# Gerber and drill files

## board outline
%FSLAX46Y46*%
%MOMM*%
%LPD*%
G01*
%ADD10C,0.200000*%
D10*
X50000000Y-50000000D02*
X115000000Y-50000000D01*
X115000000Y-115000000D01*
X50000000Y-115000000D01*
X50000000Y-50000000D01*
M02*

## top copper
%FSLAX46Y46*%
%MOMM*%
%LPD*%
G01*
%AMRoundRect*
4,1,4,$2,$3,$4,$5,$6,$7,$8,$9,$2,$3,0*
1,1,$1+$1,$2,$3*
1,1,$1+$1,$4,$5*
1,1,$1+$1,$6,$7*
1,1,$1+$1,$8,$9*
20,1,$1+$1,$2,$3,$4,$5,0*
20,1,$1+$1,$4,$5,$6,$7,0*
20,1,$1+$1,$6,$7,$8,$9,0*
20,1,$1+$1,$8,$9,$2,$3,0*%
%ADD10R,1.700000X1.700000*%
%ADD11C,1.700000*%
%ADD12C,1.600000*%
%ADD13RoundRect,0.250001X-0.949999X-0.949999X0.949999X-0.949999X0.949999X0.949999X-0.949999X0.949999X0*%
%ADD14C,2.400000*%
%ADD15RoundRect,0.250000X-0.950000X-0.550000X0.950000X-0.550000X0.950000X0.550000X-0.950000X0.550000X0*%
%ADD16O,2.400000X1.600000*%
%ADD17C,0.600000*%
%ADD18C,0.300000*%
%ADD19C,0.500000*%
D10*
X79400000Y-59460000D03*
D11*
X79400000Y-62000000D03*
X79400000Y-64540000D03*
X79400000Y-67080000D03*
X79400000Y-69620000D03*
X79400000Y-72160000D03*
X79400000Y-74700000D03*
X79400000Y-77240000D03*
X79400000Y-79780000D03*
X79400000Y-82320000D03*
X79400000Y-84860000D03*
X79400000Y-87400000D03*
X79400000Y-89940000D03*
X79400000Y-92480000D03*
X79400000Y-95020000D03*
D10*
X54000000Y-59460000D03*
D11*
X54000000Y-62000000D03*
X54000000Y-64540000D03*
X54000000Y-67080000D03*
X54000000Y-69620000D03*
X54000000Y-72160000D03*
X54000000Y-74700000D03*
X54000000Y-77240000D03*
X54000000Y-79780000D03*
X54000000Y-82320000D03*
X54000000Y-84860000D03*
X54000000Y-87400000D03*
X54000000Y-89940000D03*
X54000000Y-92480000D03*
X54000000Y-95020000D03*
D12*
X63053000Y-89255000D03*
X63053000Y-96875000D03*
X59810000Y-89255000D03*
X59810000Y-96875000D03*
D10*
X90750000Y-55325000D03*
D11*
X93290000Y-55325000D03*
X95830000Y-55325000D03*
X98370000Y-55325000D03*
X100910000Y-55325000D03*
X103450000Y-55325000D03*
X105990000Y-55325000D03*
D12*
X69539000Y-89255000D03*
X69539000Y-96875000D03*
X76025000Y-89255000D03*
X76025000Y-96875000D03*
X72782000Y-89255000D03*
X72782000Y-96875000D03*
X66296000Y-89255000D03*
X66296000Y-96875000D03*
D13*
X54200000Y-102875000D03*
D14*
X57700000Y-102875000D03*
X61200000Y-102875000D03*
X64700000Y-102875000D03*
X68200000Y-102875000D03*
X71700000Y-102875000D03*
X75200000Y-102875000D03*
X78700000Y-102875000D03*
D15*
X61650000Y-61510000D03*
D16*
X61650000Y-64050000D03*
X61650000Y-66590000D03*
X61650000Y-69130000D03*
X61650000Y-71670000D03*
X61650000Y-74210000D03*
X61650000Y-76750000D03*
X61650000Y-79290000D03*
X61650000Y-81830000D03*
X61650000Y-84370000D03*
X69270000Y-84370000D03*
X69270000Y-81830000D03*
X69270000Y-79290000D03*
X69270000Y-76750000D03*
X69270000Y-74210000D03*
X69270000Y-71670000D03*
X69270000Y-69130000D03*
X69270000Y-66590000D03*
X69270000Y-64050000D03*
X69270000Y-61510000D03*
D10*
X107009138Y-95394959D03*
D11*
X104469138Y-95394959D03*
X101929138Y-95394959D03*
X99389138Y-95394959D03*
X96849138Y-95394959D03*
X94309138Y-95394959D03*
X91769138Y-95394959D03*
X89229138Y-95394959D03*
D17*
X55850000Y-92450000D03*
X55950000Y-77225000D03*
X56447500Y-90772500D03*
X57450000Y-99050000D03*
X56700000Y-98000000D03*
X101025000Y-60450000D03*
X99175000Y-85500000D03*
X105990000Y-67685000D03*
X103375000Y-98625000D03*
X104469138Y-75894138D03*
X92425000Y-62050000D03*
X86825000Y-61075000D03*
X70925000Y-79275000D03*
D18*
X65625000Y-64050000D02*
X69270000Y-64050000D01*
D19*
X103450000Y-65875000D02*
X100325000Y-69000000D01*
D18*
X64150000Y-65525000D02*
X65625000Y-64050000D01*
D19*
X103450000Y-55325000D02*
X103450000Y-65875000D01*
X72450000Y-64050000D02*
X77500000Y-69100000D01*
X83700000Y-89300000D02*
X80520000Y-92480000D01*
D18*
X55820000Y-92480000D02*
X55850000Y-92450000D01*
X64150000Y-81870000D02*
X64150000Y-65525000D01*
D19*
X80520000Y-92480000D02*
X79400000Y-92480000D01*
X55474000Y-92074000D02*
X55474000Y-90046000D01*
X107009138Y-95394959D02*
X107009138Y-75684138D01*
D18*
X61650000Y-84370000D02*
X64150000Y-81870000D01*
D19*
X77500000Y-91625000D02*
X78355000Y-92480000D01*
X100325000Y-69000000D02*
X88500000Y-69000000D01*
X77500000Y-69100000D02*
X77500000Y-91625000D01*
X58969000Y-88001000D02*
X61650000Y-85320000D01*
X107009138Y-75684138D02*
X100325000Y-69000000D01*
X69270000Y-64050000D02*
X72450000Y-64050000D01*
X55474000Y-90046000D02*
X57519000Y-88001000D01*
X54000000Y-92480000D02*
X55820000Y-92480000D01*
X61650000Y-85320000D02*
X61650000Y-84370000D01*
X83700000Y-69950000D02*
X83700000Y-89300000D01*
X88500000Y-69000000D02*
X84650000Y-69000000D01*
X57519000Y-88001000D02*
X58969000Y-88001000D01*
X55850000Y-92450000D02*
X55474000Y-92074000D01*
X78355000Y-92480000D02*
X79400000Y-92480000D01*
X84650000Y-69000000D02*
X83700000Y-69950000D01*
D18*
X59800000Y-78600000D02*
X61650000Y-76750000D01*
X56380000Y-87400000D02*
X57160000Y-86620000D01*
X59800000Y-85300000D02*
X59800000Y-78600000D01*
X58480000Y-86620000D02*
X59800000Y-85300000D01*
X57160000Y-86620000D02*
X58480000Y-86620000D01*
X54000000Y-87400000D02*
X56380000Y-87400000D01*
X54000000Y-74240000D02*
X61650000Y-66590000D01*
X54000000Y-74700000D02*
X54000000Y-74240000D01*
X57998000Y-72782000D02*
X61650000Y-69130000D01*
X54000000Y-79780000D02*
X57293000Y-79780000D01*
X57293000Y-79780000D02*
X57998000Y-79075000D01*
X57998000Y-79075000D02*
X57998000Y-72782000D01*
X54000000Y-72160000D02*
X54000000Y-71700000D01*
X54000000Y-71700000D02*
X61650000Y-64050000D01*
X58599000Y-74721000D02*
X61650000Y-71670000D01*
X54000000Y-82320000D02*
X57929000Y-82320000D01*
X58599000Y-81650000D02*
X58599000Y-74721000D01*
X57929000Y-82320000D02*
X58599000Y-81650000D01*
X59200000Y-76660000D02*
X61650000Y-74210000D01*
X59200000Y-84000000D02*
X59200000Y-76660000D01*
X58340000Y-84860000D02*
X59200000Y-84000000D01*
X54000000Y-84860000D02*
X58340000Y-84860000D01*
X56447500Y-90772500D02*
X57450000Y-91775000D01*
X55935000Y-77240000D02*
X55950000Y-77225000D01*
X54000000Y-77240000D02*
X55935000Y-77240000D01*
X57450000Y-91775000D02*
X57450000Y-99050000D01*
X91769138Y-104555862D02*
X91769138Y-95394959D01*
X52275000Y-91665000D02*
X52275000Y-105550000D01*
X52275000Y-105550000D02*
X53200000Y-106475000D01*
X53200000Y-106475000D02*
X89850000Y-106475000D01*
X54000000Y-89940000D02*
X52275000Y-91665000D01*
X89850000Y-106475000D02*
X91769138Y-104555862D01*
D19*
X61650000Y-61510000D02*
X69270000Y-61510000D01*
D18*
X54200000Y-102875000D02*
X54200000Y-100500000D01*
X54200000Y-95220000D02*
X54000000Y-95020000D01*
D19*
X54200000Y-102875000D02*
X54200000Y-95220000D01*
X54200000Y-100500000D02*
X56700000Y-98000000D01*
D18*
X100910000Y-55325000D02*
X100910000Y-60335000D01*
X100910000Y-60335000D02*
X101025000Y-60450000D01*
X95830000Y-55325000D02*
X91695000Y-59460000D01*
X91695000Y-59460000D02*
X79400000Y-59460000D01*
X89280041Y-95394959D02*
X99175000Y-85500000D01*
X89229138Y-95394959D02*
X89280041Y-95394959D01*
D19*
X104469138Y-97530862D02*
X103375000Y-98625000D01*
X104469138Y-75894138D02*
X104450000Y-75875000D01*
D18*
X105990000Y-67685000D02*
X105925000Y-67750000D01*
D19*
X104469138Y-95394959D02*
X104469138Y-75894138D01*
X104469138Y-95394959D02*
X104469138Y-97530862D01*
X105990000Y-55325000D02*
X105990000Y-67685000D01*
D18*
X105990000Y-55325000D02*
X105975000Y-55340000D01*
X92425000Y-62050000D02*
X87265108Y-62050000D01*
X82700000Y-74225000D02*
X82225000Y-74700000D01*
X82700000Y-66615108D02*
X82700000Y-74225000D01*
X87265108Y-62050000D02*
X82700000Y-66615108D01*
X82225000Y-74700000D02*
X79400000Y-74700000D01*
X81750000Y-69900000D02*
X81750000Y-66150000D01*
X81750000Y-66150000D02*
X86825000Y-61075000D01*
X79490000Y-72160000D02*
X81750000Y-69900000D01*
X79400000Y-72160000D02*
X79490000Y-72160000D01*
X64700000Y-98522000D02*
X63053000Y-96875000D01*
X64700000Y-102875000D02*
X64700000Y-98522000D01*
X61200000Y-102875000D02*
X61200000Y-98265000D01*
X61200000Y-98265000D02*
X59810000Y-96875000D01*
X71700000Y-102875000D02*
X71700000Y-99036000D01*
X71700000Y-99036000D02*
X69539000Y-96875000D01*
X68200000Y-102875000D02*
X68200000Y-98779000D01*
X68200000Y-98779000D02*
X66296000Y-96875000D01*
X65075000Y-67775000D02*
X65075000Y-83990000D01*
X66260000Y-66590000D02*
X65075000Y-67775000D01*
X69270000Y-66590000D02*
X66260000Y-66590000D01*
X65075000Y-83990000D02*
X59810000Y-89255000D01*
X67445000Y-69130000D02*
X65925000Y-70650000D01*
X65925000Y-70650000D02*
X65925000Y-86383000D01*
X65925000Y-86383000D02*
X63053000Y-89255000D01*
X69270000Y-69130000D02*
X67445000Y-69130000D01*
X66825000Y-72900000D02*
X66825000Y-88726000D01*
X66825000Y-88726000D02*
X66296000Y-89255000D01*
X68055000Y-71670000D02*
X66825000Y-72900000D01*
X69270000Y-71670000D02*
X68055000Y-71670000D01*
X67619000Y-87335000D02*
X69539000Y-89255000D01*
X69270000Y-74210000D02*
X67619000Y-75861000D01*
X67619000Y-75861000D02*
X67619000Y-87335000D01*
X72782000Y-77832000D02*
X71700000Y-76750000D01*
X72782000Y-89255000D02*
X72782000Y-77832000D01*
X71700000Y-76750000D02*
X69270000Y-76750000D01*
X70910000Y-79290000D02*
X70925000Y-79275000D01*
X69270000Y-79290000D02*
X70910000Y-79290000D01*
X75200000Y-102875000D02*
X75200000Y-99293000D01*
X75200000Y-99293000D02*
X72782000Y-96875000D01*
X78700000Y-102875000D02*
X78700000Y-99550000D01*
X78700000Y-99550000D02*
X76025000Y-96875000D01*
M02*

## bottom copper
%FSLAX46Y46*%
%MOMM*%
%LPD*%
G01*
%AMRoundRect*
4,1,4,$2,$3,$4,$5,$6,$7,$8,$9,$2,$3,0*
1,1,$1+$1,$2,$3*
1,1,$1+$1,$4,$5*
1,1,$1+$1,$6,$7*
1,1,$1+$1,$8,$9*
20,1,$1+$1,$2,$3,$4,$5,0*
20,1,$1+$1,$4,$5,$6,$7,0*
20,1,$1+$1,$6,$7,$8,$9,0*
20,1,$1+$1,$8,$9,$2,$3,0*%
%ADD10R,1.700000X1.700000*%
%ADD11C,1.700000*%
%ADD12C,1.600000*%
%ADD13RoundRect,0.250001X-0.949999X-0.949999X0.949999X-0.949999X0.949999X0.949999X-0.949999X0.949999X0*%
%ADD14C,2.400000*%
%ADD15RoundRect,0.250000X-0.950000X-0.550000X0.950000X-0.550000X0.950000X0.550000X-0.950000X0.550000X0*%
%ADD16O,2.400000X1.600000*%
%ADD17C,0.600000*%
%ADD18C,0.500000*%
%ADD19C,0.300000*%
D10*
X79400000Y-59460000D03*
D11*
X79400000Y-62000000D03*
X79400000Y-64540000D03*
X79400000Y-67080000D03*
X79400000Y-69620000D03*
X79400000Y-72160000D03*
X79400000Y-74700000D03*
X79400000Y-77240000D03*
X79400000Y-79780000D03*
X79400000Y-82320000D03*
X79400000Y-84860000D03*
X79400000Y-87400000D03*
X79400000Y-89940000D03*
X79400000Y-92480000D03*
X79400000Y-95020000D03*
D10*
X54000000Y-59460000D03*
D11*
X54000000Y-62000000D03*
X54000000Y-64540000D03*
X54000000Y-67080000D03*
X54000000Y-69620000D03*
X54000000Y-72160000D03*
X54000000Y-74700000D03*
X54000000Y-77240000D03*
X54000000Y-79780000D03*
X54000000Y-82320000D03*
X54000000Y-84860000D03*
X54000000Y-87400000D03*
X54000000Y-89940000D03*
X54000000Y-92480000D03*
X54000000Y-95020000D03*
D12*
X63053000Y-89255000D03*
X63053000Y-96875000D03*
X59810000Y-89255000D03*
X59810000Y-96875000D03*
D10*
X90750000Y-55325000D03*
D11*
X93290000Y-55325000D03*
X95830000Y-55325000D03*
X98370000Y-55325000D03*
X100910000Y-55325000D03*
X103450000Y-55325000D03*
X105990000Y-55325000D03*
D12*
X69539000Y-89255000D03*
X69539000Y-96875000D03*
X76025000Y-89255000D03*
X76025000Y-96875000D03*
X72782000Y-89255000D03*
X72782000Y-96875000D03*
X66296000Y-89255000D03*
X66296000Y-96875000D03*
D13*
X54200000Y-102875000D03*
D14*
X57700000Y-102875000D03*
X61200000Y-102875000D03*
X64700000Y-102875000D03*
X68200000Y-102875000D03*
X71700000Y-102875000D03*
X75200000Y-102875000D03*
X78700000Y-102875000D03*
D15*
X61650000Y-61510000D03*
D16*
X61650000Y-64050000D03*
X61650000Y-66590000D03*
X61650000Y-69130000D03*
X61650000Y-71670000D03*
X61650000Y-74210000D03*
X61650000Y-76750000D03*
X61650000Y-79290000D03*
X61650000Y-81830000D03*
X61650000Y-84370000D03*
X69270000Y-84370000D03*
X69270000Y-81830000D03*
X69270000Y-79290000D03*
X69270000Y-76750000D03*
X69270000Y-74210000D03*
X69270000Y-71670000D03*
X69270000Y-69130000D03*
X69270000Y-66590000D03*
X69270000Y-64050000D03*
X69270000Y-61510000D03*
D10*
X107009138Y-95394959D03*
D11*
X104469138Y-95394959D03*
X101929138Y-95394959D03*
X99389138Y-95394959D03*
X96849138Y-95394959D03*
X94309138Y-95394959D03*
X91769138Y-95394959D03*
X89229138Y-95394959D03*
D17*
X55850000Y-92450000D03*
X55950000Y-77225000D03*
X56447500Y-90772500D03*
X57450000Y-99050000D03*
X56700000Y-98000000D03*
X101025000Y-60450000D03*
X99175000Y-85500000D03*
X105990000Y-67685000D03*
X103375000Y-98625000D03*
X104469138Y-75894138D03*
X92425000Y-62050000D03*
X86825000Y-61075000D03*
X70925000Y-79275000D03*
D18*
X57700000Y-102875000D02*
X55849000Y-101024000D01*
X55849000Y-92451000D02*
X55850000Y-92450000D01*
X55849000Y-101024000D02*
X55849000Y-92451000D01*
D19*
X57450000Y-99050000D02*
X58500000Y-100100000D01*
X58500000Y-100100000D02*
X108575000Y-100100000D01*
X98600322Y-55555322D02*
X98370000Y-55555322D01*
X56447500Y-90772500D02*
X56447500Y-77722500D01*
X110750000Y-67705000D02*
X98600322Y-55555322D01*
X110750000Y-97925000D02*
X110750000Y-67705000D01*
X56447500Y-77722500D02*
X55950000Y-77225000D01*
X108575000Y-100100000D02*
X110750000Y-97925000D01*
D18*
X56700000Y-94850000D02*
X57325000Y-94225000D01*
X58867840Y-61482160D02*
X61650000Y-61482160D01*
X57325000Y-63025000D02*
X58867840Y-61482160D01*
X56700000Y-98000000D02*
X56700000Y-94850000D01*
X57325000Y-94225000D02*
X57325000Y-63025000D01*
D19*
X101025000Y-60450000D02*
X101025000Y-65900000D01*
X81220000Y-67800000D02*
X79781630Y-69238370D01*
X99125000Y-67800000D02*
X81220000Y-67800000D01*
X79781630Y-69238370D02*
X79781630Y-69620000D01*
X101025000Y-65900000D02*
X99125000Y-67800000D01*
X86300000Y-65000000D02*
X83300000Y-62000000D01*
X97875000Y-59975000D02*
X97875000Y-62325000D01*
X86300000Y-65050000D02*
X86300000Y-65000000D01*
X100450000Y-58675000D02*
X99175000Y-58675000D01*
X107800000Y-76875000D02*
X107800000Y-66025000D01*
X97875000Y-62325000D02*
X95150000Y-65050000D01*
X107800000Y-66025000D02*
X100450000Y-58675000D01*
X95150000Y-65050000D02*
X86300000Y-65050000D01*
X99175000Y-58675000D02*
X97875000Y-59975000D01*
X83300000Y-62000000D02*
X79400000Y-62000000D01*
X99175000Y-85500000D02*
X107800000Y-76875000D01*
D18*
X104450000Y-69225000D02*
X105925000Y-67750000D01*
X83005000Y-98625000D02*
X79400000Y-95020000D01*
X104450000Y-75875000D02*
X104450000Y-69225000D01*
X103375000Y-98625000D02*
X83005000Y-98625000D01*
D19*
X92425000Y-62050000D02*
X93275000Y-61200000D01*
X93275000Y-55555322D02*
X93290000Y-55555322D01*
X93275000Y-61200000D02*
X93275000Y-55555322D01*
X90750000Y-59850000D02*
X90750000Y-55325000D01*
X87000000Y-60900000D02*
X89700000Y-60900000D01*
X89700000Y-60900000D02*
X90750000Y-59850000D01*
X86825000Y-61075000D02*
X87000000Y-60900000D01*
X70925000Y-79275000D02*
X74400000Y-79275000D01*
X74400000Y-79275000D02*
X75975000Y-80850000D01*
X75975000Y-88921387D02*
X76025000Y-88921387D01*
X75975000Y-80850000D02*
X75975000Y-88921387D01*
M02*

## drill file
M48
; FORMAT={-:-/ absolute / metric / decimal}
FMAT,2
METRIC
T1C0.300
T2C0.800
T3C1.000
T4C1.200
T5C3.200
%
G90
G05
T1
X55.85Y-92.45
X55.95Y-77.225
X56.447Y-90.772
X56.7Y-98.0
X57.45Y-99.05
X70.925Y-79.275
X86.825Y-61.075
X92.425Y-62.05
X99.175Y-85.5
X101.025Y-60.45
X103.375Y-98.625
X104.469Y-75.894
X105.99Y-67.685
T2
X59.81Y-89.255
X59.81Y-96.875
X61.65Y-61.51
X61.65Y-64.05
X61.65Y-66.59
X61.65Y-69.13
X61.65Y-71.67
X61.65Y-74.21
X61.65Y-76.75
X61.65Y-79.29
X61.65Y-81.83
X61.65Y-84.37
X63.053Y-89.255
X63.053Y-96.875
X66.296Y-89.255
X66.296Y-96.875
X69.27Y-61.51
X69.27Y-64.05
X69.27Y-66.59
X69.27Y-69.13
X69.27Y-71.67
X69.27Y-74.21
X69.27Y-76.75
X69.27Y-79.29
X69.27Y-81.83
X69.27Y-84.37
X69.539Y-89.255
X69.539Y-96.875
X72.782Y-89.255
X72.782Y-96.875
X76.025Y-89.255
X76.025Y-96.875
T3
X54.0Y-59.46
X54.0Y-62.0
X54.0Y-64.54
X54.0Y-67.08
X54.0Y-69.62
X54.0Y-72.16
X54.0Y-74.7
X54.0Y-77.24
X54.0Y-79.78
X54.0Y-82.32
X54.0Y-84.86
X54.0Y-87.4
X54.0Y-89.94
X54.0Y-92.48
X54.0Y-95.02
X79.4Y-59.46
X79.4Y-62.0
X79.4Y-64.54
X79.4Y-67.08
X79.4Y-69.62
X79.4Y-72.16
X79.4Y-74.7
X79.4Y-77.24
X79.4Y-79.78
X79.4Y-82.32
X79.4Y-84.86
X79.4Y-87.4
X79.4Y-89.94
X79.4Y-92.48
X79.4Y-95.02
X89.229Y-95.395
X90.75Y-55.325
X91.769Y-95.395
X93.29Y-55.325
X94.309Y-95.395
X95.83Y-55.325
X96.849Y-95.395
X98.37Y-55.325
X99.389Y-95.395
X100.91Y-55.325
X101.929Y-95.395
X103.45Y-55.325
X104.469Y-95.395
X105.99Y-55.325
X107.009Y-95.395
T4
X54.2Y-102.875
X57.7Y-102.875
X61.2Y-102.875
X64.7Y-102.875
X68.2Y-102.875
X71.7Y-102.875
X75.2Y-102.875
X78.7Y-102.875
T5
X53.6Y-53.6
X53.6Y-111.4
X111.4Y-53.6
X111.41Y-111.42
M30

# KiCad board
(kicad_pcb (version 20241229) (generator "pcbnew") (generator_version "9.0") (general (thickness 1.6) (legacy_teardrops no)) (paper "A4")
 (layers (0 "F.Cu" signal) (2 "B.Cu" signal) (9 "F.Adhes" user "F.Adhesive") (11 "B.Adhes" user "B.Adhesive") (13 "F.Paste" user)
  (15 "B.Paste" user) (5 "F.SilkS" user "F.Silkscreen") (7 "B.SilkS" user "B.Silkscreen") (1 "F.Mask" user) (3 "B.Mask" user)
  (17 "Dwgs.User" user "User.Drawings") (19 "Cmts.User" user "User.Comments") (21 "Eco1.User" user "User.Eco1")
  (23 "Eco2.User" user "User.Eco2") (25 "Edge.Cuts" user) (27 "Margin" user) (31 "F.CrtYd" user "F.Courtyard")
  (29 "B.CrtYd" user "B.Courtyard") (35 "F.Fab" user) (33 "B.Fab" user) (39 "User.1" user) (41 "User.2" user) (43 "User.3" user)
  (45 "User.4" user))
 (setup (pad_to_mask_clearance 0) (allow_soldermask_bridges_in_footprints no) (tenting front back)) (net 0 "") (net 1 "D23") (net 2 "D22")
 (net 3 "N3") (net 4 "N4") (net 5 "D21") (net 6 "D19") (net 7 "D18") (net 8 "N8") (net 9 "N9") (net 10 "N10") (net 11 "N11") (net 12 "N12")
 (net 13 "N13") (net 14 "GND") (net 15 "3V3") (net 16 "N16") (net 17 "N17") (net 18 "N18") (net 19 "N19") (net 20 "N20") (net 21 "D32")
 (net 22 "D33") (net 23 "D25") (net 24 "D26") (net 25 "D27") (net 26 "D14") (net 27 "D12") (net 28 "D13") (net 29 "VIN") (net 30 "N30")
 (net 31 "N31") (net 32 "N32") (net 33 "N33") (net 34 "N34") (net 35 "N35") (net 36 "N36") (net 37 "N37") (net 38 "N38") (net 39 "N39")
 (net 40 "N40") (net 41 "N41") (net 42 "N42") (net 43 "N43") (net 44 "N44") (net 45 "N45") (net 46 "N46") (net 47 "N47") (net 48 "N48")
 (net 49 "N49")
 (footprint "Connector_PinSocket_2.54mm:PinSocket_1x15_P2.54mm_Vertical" (layer "F.Cu") (at 79.4 59.46)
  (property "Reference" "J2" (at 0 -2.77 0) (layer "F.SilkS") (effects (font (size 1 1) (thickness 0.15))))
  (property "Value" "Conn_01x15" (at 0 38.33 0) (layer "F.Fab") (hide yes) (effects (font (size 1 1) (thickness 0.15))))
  (pad "1" thru_hole rect (at 0 0) (size 1.7 1.7) (drill 1) (layers "*.Cu" "*.Mask") (remove_unused_layers no) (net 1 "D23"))
  (pad "2" thru_hole circle (at 0 2.54) (size 1.7 1.7) (drill 1) (layers "*.Cu" "*.Mask") (remove_unused_layers no) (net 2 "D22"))
  (pad "3" thru_hole circle (at 0 5.08) (size 1.7 1.7) (drill 1) (layers "*.Cu" "*.Mask") (remove_unused_layers no) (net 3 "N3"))
  (pad "4" thru_hole circle (at 0 7.62) (size 1.7 1.7) (drill 1) (layers "*.Cu" "*.Mask") (remove_unused_layers no) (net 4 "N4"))
  (pad "5" thru_hole circle (at 0 10.16) (size 1.7 1.7) (drill 1) (layers "*.Cu" "*.Mask") (remove_unused_layers no) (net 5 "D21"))
  (pad "6" thru_hole circle (at 0 12.7) (size 1.7 1.7) (drill 1) (layers "*.Cu" "*.Mask") (remove_unused_layers no) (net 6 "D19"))
  (pad "7" thru_hole circle (at 0 15.24) (size 1.7 1.7) (drill 1) (layers "*.Cu" "*.Mask") (remove_unused_layers no) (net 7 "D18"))
  (pad "8" thru_hole circle (at 0 17.78) (size 1.7 1.7) (drill 1) (layers "*.Cu" "*.Mask") (remove_unused_layers no) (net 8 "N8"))
  (pad "9" thru_hole circle (at 0 20.32) (size 1.7 1.7) (drill 1) (layers "*.Cu" "*.Mask") (remove_unused_layers no) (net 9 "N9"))
  (pad "10" thru_hole circle (at 0 22.86) (size 1.7 1.7) (drill 1) (layers "*.Cu" "*.Mask") (remove_unused_layers no) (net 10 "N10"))
  (pad "11" thru_hole circle (at 0 25.4) (size 1.7 1.7) (drill 1) (layers "*.Cu" "*.Mask") (remove_unused_layers no) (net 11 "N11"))
  (pad "12" thru_hole circle (at 0 27.94) (size 1.7 1.7) (drill 1) (layers "*.Cu" "*.Mask") (remove_unused_layers no) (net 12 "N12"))
  (pad "13" thru_hole circle (at 0 30.48) (size 1.7 1.7) (drill 1) (layers "*.Cu" "*.Mask") (remove_unused_layers no) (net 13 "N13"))
  (pad "14" thru_hole circle (at 0 33.02) (size 1.7 1.7) (drill 1) (layers "*.Cu" "*.Mask") (remove_unused_layers no) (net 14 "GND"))
  (pad "15" thru_hole circle (at 0 35.56) (size 1.7 1.7) (drill 1) (layers "*.Cu" "*.Mask") (remove_unused_layers no) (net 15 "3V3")))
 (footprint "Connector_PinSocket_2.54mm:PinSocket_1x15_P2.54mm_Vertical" (layer "F.Cu") (at 54 59.46)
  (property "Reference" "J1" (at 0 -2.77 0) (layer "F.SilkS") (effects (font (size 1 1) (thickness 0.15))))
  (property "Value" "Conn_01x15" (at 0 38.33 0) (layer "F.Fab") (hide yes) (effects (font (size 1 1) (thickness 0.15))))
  (pad "1" thru_hole rect (at 0 0) (size 1.7 1.7) (drill 1) (layers "*.Cu" "*.Mask") (remove_unused_layers no) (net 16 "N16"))
  (pad "2" thru_hole circle (at 0 2.54) (size 1.7 1.7) (drill 1) (layers "*.Cu" "*.Mask") (remove_unused_layers no) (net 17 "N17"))
  (pad "3" thru_hole circle (at 0 5.08) (size 1.7 1.7) (drill 1) (layers "*.Cu" "*.Mask") (remove_unused_layers no) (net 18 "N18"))
  (pad "4" thru_hole circle (at 0 7.62) (size 1.7 1.7) (drill 1) (layers "*.Cu" "*.Mask") (remove_unused_layers no) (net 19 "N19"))
  (pad "5" thru_hole circle (at 0 10.16) (size 1.7 1.7) (drill 1) (layers "*.Cu" "*.Mask") (remove_unused_layers no) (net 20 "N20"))
  (pad "6" thru_hole circle (at 0 12.7) (size 1.7 1.7) (drill 1) (layers "*.Cu" "*.Mask") (remove_unused_layers no) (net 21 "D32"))
  (pad "7" thru_hole circle (at 0 15.24) (size 1.7 1.7) (drill 1) (layers "*.Cu" "*.Mask") (remove_unused_layers no) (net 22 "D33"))
  (pad "8" thru_hole circle (at 0 17.78) (size 1.7 1.7) (drill 1) (layers "*.Cu" "*.Mask") (remove_unused_layers no) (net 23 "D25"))
  (pad "9" thru_hole circle (at 0 20.32) (size 1.7 1.7) (drill 1) (layers "*.Cu" "*.Mask") (remove_unused_layers no) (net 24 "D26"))
  (pad "10" thru_hole circle (at 0 22.86) (size 1.7 1.7) (drill 1) (layers "*.Cu" "*.Mask") (remove_unused_layers no) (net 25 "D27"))
  (pad "11" thru_hole circle (at 0 25.4) (size 1.7 1.7) (drill 1) (layers "*.Cu" "*.Mask") (remove_unused_layers no) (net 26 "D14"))
  (pad "12" thru_hole circle (at 0 27.94) (size 1.7 1.7) (drill 1) (layers "*.Cu" "*.Mask") (remove_unused_layers no) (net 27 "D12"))
  (pad "13" thru_hole circle (at 0 30.48) (size 1.7 1.7) (drill 1) (layers "*.Cu" "*.Mask") (remove_unused_layers no) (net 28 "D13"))
  (pad "14" thru_hole circle (at 0 33.02) (size 1.7 1.7) (drill 1) (layers "*.Cu" "*.Mask") (remove_unused_layers no) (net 14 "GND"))
  (pad "15" thru_hole circle (at 0 35.56) (size 1.7 1.7) (drill 1) (layers "*.Cu" "*.Mask") (remove_unused_layers no) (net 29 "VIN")))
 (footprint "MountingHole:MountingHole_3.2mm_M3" (layer "F.Cu") (at 53.6 53.6)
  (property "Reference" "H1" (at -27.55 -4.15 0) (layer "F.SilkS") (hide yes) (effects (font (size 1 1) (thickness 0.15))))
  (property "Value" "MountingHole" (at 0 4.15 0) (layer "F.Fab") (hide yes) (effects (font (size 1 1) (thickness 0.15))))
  (pad "" np_thru_hole circle (at 0 0) (size 3.2 3.2) (drill 3.2) (layers "*.Cu" "*.Mask")))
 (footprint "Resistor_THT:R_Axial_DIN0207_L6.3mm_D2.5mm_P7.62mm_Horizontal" (layer "F.Cu") (at 63.053 89.255 -90)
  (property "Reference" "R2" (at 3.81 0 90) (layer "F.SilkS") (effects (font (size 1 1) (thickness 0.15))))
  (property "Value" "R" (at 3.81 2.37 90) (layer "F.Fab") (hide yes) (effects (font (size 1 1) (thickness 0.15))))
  (pad "1" thru_hole circle (at 0 0 270) (size 1.6 1.6) (drill 0.8) (layers "*.Cu" "*.Mask") (remove_unused_layers no) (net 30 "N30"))
  (pad "2" thru_hole circle (at 7.62 0 270) (size 1.6 1.6) (drill 0.8) (layers "*.Cu" "*.Mask") (remove_unused_layers no) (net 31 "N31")))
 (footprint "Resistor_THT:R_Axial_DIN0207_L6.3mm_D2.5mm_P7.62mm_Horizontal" (layer "F.Cu") (at 59.81 89.255 -90)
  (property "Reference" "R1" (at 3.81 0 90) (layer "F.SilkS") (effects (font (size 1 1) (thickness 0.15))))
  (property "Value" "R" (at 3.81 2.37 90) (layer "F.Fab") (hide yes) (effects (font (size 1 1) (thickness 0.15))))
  (pad "1" thru_hole circle (at 0 0 270) (size 1.6 1.6) (drill 0.8) (layers "*.Cu" "*.Mask") (remove_unused_layers no) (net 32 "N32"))
  (pad "2" thru_hole circle (at 7.62 0 270) (size 1.6 1.6) (drill 0.8) (layers "*.Cu" "*.Mask") (remove_unused_layers no) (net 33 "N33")))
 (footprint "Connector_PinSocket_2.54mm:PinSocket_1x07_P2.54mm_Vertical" (layer "F.Cu") (at 90.75 55.325 90)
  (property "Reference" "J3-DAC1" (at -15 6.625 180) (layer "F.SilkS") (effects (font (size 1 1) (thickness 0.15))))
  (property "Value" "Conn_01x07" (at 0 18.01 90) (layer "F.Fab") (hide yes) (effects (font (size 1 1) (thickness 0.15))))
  (pad "1" thru_hole rect (at 0 0 90) (size 1.7 1.7) (drill 1) (layers "*.Cu" "*.Mask") (remove_unused_layers no) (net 6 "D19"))
  (pad "2" thru_hole circle (at 0 2.54 90) (size 1.7 1.7) (drill 1) (layers "*.Cu" "*.Mask") (remove_unused_layers no) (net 7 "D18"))
  (pad "3" thru_hole circle (at 0 5.08 90) (size 1.7 1.7) (drill 1) (layers "*.Cu" "*.Mask") (remove_unused_layers no) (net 1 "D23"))
  (pad "4" thru_hole circle (at 0 7.62 90) (size 1.7 1.7) (drill 1) (layers "*.Cu" "*.Mask") (remove_unused_layers no) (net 23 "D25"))
  (pad "5" thru_hole circle (at 0 10.16 90) (size 1.7 1.7) (drill 1) (layers "*.Cu" "*.Mask") (remove_unused_layers no) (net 5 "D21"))
  (pad "6" thru_hole circle (at 0 12.7 90) (size 1.7 1.7) (drill 1) (layers "*.Cu" "*.Mask") (remove_unused_layers no) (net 14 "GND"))
  (pad "7" thru_hole circle (at 0 15.24 90) (size 1.7 1.7) (drill 1) (layers "*.Cu" "*.Mask") (remove_unused_layers no) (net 15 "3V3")))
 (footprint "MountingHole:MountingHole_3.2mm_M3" (layer "F.Cu") (at 53.6 111.4)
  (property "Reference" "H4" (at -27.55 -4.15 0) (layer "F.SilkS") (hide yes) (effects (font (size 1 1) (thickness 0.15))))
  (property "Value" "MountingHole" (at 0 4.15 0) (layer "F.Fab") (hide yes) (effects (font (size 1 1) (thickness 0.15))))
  (pad "" np_thru_hole circle (at 0 0) (size 3.2 3.2) (drill 3.2) (layers "*.Cu" "*.Mask")))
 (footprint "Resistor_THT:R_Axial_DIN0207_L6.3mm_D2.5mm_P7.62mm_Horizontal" (layer "F.Cu") (at 69.539 89.255 -90)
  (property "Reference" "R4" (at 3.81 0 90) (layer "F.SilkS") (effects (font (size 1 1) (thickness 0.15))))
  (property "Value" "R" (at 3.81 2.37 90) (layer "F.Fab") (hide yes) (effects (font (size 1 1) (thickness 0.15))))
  (pad "1" thru_hole circle (at 0 0 270) (size 1.6 1.6) (drill 0.8) (layers "*.Cu" "*.Mask") (remove_unused_layers no) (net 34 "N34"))
  (pad "2" thru_hole circle (at 7.62 0 270) (size 1.6 1.6) (drill 0.8) (layers "*.Cu" "*.Mask") (remove_unused_layers no) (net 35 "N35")))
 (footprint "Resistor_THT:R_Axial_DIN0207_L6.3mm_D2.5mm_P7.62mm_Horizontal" (layer "F.Cu") (at 76.025 89.255 -90)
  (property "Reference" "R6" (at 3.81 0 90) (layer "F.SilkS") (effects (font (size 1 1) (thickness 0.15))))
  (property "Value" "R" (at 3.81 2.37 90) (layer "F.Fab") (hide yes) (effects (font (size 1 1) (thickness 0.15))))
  (pad "1" thru_hole circle (at 0 0 270) (size 1.6 1.6) (drill 0.8) (layers "*.Cu" "*.Mask") (remove_unused_layers no) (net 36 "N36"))
  (pad "2" thru_hole circle (at 7.62 0 270) (size 1.6 1.6) (drill 0.8) (layers "*.Cu" "*.Mask") (remove_unused_layers no) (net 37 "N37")))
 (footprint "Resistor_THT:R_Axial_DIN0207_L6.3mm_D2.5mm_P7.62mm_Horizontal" (layer "F.Cu") (at 72.782 89.255 -90)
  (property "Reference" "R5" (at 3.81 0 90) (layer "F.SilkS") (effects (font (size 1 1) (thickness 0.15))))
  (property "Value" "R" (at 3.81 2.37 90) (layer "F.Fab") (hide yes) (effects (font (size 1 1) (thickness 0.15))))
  (pad "1" thru_hole circle (at 0 0 270) (size 1.6 1.6) (drill 0.8) (layers "*.Cu" "*.Mask") (remove_unused_layers no) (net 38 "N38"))
  (pad "2" thru_hole circle (at 7.62 0 270) (size 1.6 1.6) (drill 0.8) (layers "*.Cu" "*.Mask") (remove_unused_layers no) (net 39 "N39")))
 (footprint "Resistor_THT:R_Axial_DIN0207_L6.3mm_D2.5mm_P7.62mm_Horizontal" (layer "F.Cu") (at 66.296 89.255 -90)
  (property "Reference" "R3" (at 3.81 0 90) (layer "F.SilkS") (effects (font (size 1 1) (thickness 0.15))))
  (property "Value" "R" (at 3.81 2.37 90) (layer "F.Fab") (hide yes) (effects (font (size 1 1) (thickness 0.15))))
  (pad "1" thru_hole circle (at 0 0 270) (size 1.6 1.6) (drill 0.8) (layers "*.Cu" "*.Mask") (remove_unused_layers no) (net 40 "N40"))
  (pad "2" thru_hole circle (at 7.62 0 270) (size 1.6 1.6) (drill 0.8) (layers "*.Cu" "*.Mask") (remove_unused_layers no) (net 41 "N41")))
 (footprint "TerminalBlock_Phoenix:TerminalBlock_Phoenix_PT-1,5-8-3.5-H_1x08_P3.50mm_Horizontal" (layer "F.Cu") (at 54.2 102.875)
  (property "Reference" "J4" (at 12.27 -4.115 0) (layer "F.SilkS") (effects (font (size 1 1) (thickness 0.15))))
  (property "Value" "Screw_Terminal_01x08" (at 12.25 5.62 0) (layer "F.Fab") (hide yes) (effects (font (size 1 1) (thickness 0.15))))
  (pad "1" thru_hole roundrect (at 0 0) (size 2.4 2.4) (drill 1.2) (layers "*.Cu" "*.Mask") (remove_unused_layers no)
   (roundrect_rratio 0.104167) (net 29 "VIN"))
  (pad "2" thru_hole circle (at 3.5 0) (size 2.4 2.4) (drill 1.2) (layers "*.Cu" "*.Mask") (remove_unused_layers no) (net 14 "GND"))
  (pad "3" thru_hole circle (at 7 0) (size 2.4 2.4) (drill 1.2) (layers "*.Cu" "*.Mask") (remove_unused_layers no) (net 33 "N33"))
  (pad "4" thru_hole circle (at 10.5 0) (size 2.4 2.4) (drill 1.2) (layers "*.Cu" "*.Mask") (remove_unused_layers no) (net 31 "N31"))
  (pad "5" thru_hole circle (at 14 0) (size 2.4 2.4) (drill 1.2) (layers "*.Cu" "*.Mask") (remove_unused_layers no) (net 41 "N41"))
  (pad "6" thru_hole circle (at 17.5 0) (size 2.4 2.4) (drill 1.2) (layers "*.Cu" "*.Mask") (remove_unused_layers no) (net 35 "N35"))
  (pad "7" thru_hole circle (at 21 0) (size 2.4 2.4) (drill 1.2) (layers "*.Cu" "*.Mask") (remove_unused_layers no) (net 39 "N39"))
  (pad "8" thru_hole circle (at 24.5 0) (size 2.4 2.4) (drill 1.2) (layers "*.Cu" "*.Mask") (remove_unused_layers no) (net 37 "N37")))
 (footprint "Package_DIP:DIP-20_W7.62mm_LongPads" (layer "F.Cu") (at 61.65 61.51)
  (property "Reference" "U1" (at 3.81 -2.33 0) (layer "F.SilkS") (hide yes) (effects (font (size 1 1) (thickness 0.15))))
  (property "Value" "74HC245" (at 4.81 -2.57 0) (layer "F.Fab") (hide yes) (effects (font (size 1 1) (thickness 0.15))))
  (pad "1" thru_hole roundrect (at 0 0) (size 2.4 1.6) (drill 0.8) (layers "*.Cu" "*.Mask") (remove_unused_layers no)
   (roundrect_rratio 0.15625) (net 29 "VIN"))
  (pad "2" thru_hole oval (at 0 2.54) (size 2.4 1.6) (drill 0.8) (layers "*.Cu" "*.Mask") (remove_unused_layers no) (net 21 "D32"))
  (pad "3" thru_hole oval (at 0 5.08) (size 2.4 1.6) (drill 0.8) (layers "*.Cu" "*.Mask") (remove_unused_layers no) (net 22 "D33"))
  (pad "4" thru_hole oval (at 0 7.62) (size 2.4 1.6) (drill 0.8) (layers "*.Cu" "*.Mask") (remove_unused_layers no) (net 24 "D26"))
  (pad "5" thru_hole oval (at 0 10.16) (size 2.4 1.6) (drill 0.8) (layers "*.Cu" "*.Mask") (remove_unused_layers no) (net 25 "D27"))
  (pad "6" thru_hole oval (at 0 12.7) (size 2.4 1.6) (drill 0.8) (layers "*.Cu" "*.Mask") (remove_unused_layers no) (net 26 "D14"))
  (pad "7" thru_hole oval (at 0 15.24) (size 2.4 1.6) (drill 0.8) (layers "*.Cu" "*.Mask") (remove_unused_layers no) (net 27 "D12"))
  (pad "8" thru_hole oval (at 0 17.78) (size 2.4 1.6) (drill 0.8) (layers "*.Cu" "*.Mask") (remove_unused_layers no) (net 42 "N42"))
  (pad "9" thru_hole oval (at 0 20.32) (size 2.4 1.6) (drill 0.8) (layers "*.Cu" "*.Mask") (remove_unused_layers no) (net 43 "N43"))
  (pad "10" thru_hole oval (at 0 22.86) (size 2.4 1.6) (drill 0.8) (layers "*.Cu" "*.Mask") (remove_unused_layers no) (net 14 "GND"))
  (pad "11" thru_hole oval (at 7.62 22.86) (size 2.4 1.6) (drill 0.8) (layers "*.Cu" "*.Mask") (remove_unused_layers no) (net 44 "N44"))
  (pad "12" thru_hole oval (at 7.62 20.32) (size 2.4 1.6) (drill 0.8) (layers "*.Cu" "*.Mask") (remove_unused_layers no) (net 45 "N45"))
  (pad "13" thru_hole oval (at 7.62 17.78) (size 2.4 1.6) (drill 0.8) (layers "*.Cu" "*.Mask") (remove_unused_layers no) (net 36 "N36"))
  (pad "14" thru_hole oval (at 7.62 15.24) (size 2.4 1.6) (drill 0.8) (layers "*.Cu" "*.Mask") (remove_unused_layers no) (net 38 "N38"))
  (pad "15" thru_hole oval (at 7.62 12.7) (size 2.4 1.6) (drill 0.8) (layers "*.Cu" "*.Mask") (remove_unused_layers no) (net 34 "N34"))
  (pad "16" thru_hole oval (at 7.62 10.16) (size 2.4 1.6) (drill 0.8) (layers "*.Cu" "*.Mask") (remove_unused_layers no) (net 40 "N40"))
  (pad "17" thru_hole oval (at 7.62 7.62) (size 2.4 1.6) (drill 0.8) (layers "*.Cu" "*.Mask") (remove_unused_layers no) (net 30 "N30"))
  (pad "18" thru_hole oval (at 7.62 5.08) (size 2.4 1.6) (drill 0.8) (layers "*.Cu" "*.Mask") (remove_unused_layers no) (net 32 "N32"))
  (pad "19" thru_hole oval (at 7.62 2.54) (size 2.4 1.6) (drill 0.8) (layers "*.Cu" "*.Mask") (remove_unused_layers no) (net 14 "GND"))
  (pad "20" thru_hole oval (at 7.62 0) (size 2.4 1.6) (drill 0.8) (layers "*.Cu" "*.Mask") (remove_unused_layers no) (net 29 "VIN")))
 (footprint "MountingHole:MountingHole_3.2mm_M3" (layer "F.Cu") (at 111.41 111.42)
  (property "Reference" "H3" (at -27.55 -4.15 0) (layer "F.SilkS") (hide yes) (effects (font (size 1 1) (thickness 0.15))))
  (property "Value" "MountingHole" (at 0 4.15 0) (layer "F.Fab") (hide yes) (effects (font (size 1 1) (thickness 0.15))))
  (pad "" np_thru_hole circle (at 0 0) (size 3.2 3.2) (drill 3.2) (layers "*.Cu" "*.Mask")))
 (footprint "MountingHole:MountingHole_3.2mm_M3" (layer "F.Cu") (at 111.4 53.6)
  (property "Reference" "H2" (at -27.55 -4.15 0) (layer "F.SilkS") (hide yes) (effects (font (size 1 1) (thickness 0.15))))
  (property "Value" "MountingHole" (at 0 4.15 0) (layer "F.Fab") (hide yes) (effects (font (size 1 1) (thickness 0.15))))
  (pad "" np_thru_hole circle (at 0 0) (size 3.2 3.2) (drill 3.2) (layers "*.Cu" "*.Mask")))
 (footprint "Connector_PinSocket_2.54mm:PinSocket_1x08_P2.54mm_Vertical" (layer "F.Cu") (at 107.009138 95.394959 -90)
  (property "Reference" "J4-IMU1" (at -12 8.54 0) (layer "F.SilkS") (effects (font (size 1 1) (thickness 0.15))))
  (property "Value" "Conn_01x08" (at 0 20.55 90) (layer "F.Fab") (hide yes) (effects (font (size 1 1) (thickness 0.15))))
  (pad "1" thru_hole rect (at 0 0 270) (size 1.7 1.7) (drill 1) (layers "*.Cu" "*.Mask") (remove_unused_layers no) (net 14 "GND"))
  (pad "2" thru_hole circle (at 0 2.54 270) (size 1.7 1.7) (drill 1) (layers "*.Cu" "*.Mask") (remove_unused_layers no) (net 15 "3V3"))
  (pad "3" thru_hole circle (at 0 5.08 270) (size 1.7 1.7) (drill 1) (layers "*.Cu" "*.Mask") (remove_unused_layers no) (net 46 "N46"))
  (pad "4" thru_hole circle (at 0 7.62 270) (size 1.7 1.7) (drill 1) (layers "*.Cu" "*.Mask") (remove_unused_layers no) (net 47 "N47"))
  (pad "5" thru_hole circle (at 0 10.16 270) (size 1.7 1.7) (drill 1) (layers "*.Cu" "*.Mask") (remove_unused_layers no) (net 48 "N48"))
  (pad "6" thru_hole circle (at 0 12.7 270) (size 1.7 1.7) (drill 1) (layers "*.Cu" "*.Mask") (remove_unused_layers no) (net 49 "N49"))
  (pad "7" thru_hole circle (at 0 15.24 270) (size 1.7 1.7) (drill 1) (layers "*.Cu" "*.Mask") (remove_unused_layers no) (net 28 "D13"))
  (pad "8" thru_hole circle (at 0 17.78 270) (size 1.7 1.7) (drill 1) (layers "*.Cu" "*.Mask") (remove_unused_layers no) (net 2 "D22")))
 (gr_rect (start 50 50) (end 115 115) (stroke (width 0.2) (type solid)) (fill no) (layer "Edge.Cuts"))
 (segment (start 65.625 64.05) (end 69.27 64.05) (width 0.3) (layer "F.Cu") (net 14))
 (segment (start 103.45 65.875) (end 100.325 69) (width 0.5) (layer "F.Cu") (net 14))
 (segment (start 64.15 65.525) (end 65.625 64.05) (width 0.3) (layer "F.Cu") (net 14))
 (segment (start 103.45 55.325) (end 103.45 65.875) (width 0.5) (layer "F.Cu") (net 14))
 (segment (start 72.45 64.05) (end 77.5 69.1) (width 0.5) (layer "F.Cu") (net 14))
 (segment (start 83.7 89.3) (end 80.52 92.48) (width 0.5) (layer "F.Cu") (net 14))
 (segment (start 55.82 92.48) (end 55.85 92.45) (width 0.3) (layer "F.Cu") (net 14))
 (segment (start 64.15 81.87) (end 64.15 65.525) (width 0.3) (layer "F.Cu") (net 14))
 (segment (start 80.52 92.48) (end 79.4 92.48) (width 0.5) (layer "F.Cu") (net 14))
 (segment (start 55.474 92.074) (end 55.474 90.046) (width 0.5) (layer "F.Cu") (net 14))
 (segment (start 107.009138 95.394959) (end 107.009138 75.684138) (width 0.5) (layer "F.Cu") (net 14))
 (segment (start 61.65 84.37) (end 64.15 81.87) (width 0.3) (layer "F.Cu") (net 14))
 (segment (start 77.5 91.625) (end 78.355 92.48) (width 0.5) (layer "F.Cu") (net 14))
 (segment (start 100.325 69) (end 88.5 69) (width 0.5) (layer "F.Cu") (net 14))
 (segment (start 77.5 69.1) (end 77.5 91.625) (width 0.5) (layer "F.Cu") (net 14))
 (segment (start 58.969 88.001) (end 61.65 85.32) (width 0.5) (layer "F.Cu") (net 14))
 (segment (start 107.009138 75.684138) (end 100.325 69) (width 0.5) (layer "F.Cu") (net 14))
 (segment (start 69.27 64.05) (end 72.45 64.05) (width 0.5) (layer "F.Cu") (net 14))
 (segment (start 55.474 90.046) (end 57.519 88.001) (width 0.5) (layer "F.Cu") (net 14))
 (segment (start 54 92.48) (end 55.82 92.48) (width 0.5) (layer "F.Cu") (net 14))
 (segment (start 61.65 85.32) (end 61.65 84.37) (width 0.5) (layer "F.Cu") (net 14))
 (segment (start 83.7 69.95) (end 83.7 89.3) (width 0.5) (layer "F.Cu") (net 14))
 (segment (start 88.5 69) (end 84.65 69) (width 0.5) (layer "F.Cu") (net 14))
 (segment (start 57.519 88.001) (end 58.969 88.001) (width 0.5) (layer "F.Cu") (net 14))
 (segment (start 55.85 92.45) (end 55.474 92.074) (width 0.5) (layer "F.Cu") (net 14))
 (segment (start 78.355 92.48) (end 79.4 92.48) (width 0.5) (layer "F.Cu") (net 14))
 (segment (start 84.65 69) (end 83.7 69.95) (width 0.5) (layer "F.Cu") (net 14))
 (via (at 55.85 92.45) (size 0.6) (drill 0.3) (layers "F.Cu" "B.Cu") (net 14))
 (segment (start 57.7 102.875) (end 55.849 101.024) (width 0.5) (layer "B.Cu") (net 14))
 (segment (start 55.849 92.451) (end 55.85 92.45) (width 0.5) (layer "B.Cu") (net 14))
 (segment (start 55.849 101.024) (end 55.849 92.451) (width 0.5) (layer "B.Cu") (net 14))
 (segment (start 59.8 78.6) (end 61.65 76.75) (width 0.3) (layer "F.Cu") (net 27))
 (segment (start 56.38 87.4) (end 57.16 86.62) (width 0.3) (layer "F.Cu") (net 27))
 (segment (start 59.8 85.3) (end 59.8 78.6) (width 0.3) (layer "F.Cu") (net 27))
 (segment (start 58.48 86.62) (end 59.8 85.3) (width 0.3) (layer "F.Cu") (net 27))
 (segment (start 57.16 86.62) (end 58.48 86.62) (width 0.3) (layer "F.Cu") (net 27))
 (segment (start 54 87.4) (end 56.38 87.4) (width 0.3) (layer "F.Cu") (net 27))
 (segment (start 54 74.24) (end 61.65 66.59) (width 0.3) (layer "F.Cu") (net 22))
 (segment (start 54 74.7) (end 54 74.24) (width 0.3) (layer "F.Cu") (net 22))
 (segment (start 57.998 72.782) (end 61.65 69.13) (width 0.3) (layer "F.Cu") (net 24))
 (segment (start 54 79.78) (end 57.293 79.78) (width 0.3) (layer "F.Cu") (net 24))
 (segment (start 57.293 79.78) (end 57.998 79.075) (width 0.3) (layer "F.Cu") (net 24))
 (segment (start 57.998 79.075) (end 57.998 72.782) (width 0.3) (layer "F.Cu") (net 24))
 (segment (start 54 72.16) (end 54 71.7) (width 0.3) (layer "F.Cu") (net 21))
 (segment (start 54 71.7) (end 61.65 64.05) (width 0.3) (layer "F.Cu") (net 21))
 (segment (start 58.599 74.721) (end 61.65 71.67) (width 0.3) (layer "F.Cu") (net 25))
 (segment (start 54 82.32) (end 57.929 82.32) (width 0.3) (layer "F.Cu") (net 25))
 (segment (start 58.599 81.65) (end 58.599 74.721) (width 0.3) (layer "F.Cu") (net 25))
 (segment (start 57.929 82.32) (end 58.599 81.65) (width 0.3) (layer "F.Cu") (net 25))
 (segment (start 59.2 76.66) (end 61.65 74.21) (width 0.3) (layer "F.Cu") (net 26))
 (segment (start 59.2 84) (end 59.2 76.66) (width 0.3) (layer "F.Cu") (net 26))
 (segment (start 58.34 84.86) (end 59.2 84) (width 0.3) (layer "F.Cu") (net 26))
 (segment (start 54 84.86) (end 58.34 84.86) (width 0.3) (layer "F.Cu") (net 26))
 (segment (start 56.4475 90.7725) (end 57.45 91.775) (width 0.3) (layer "F.Cu") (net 23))
 (segment (start 55.935 77.24) (end 55.95 77.225) (width 0.3) (layer "F.Cu") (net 23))
 (segment (start 54 77.24) (end 55.935 77.24) (width 0.3) (layer "F.Cu") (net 23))
 (segment (start 57.45 91.775) (end 57.45 99.05) (width 0.3) (layer "F.Cu") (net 23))
 (via (at 55.95 77.225) (size 0.6) (drill 0.3) (layers "F.Cu" "B.Cu") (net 23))
 (via (at 56.4475 90.7725) (size 0.6) (drill 0.3) (layers "F.Cu" "B.Cu") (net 23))
 (via (at 57.45 99.05) (size 0.6) (drill 0.3) (layers "F.Cu" "B.Cu") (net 23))
 (segment (start 57.45 99.05) (end 58.5 100.1) (width 0.3) (layer "B.Cu") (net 23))
 (segment (start 58.5 100.1) (end 108.575 100.1) (width 0.3) (layer "B.Cu") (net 23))
 (segment (start 98.600322 55.555322) (end 98.37 55.555322) (width 0.3) (layer "B.Cu") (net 23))
 (segment (start 56.4475 90.7725) (end 56.4475 77.7225) (width 0.3) (layer "B.Cu") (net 23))
 (segment (start 110.75 67.705) (end 98.600322 55.555322) (width 0.3) (layer "B.Cu") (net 23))
 (segment (start 110.75 97.925) (end 110.75 67.705) (width 0.3) (layer "B.Cu") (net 23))
 (segment (start 56.4475 77.7225) (end 55.95 77.225) (width 0.3) (layer "B.Cu") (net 23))
 (segment (start 108.575 100.1) (end 110.75 97.925) (width 0.3) (layer "B.Cu") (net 23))
 (segment (start 91.769138 104.555862) (end 91.769138 95.394959) (width 0.3) (layer "F.Cu") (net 28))
 (segment (start 52.275 91.665) (end 52.275 105.55) (width 0.3) (layer "F.Cu") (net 28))
 (segment (start 52.275 105.55) (end 53.2 106.475) (width 0.3) (layer "F.Cu") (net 28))
 (segment (start 53.2 106.475) (end 89.85 106.475) (width 0.3) (layer "F.Cu") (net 28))
 (segment (start 54 89.94) (end 52.275 91.665) (width 0.3) (layer "F.Cu") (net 28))
 (segment (start 89.85 106.475) (end 91.769138 104.555862) (width 0.3) (layer "F.Cu") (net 28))
 (segment (start 61.65 61.51) (end 69.27 61.51) (width 0.5) (layer "F.Cu") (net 29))
 (segment (start 54.2 102.875) (end 54.2 100.5) (width 0.3) (layer "F.Cu") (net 29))
 (segment (start 54.2 95.22) (end 54 95.02) (width 0.3) (layer "F.Cu") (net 29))
 (segment (start 54.2 102.875) (end 54.2 95.22) (width 0.5) (layer "F.Cu") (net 29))
 (segment (start 54.2 100.5) (end 56.7 98) (width 0.5) (layer "F.Cu") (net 29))
 (via (at 56.7 98) (size 0.6) (drill 0.3) (layers "F.Cu" "B.Cu") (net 29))
 (segment (start 56.7 94.85) (end 57.325 94.225) (width 0.5) (layer "B.Cu") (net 29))
 (segment (start 58.86784 61.48216) (end 61.65 61.48216) (width 0.5) (layer "B.Cu") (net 29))
 (segment (start 57.325 63.025) (end 58.86784 61.48216) (width 0.5) (layer "B.Cu") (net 29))
 (segment (start 56.7 98) (end 56.7 94.85) (width 0.5) (layer "B.Cu") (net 29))
 (segment (start 57.325 94.225) (end 57.325 63.025) (width 0.5) (layer "B.Cu") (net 29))
 (segment (start 100.91 55.325) (end 100.91 60.335) (width 0.3) (layer "F.Cu") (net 5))
 (segment (start 100.91 60.335) (end 101.025 60.45) (width 0.3) (layer "F.Cu") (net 5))
 (via (at 101.025 60.45) (size 0.6) (drill 0.3) (layers "F.Cu" "B.Cu") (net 5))
 (segment (start 101.025 60.45) (end 101.025 65.9) (width 0.3) (layer "B.Cu") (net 5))
 (segment (start 81.22 67.8) (end 79.78163 69.23837) (width 0.3) (layer "B.Cu") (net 5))
 (segment (start 99.125 67.8) (end 81.22 67.8) (width 0.3) (layer "B.Cu") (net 5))
 (segment (start 79.78163 69.23837) (end 79.78163 69.62) (width 0.3) (layer "B.Cu") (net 5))
 (segment (start 101.025 65.9) (end 99.125 67.8) (width 0.3) (layer "B.Cu") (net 5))
 (segment (start 95.83 55.325) (end 91.695 59.46) (width 0.3) (layer "F.Cu") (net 1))
 (segment (start 91.695 59.46) (end 79.4 59.46) (width 0.3) (layer "F.Cu") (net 1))
 (segment (start 89.280041 95.394959) (end 99.175 85.5) (width 0.3) (layer "F.Cu") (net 2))
 (segment (start 89.229138 95.394959) (end 89.280041 95.394959) (width 0.3) (layer "F.Cu") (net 2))
 (via (at 99.175 85.5) (size 0.6) (drill 0.3) (layers "F.Cu" "B.Cu") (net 2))
 (segment (start 86.3 65) (end 83.3 62) (width 0.3) (layer "B.Cu") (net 2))
 (segment (start 97.875 59.975) (end 97.875 62.325) (width 0.3) (layer "B.Cu") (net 2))
 (segment (start 86.3 65.05) (end 86.3 65) (width 0.3) (layer "B.Cu") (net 2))
 (segment (start 100.45 58.675) (end 99.175 58.675) (width 0.3) (layer "B.Cu") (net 2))
 (segment (start 107.8 76.875) (end 107.8 66.025) (width 0.3) (layer "B.Cu") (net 2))
 (segment (start 97.875 62.325) (end 95.15 65.05) (width 0.3) (layer "B.Cu") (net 2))
 (segment (start 107.8 66.025) (end 100.45 58.675) (width 0.3) (layer "B.Cu") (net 2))
 (segment (start 95.15 65.05) (end 86.3 65.05) (width 0.3) (layer "B.Cu") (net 2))
 (segment (start 99.175 58.675) (end 97.875 59.975) (width 0.3) (layer "B.Cu") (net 2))
 (segment (start 83.3 62) (end 79.4 62) (width 0.3) (layer "B.Cu") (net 2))
 (segment (start 99.175 85.5) (end 107.8 76.875) (width 0.3) (layer "B.Cu") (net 2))
 (segment (start 104.469138 97.530862) (end 103.375 98.625) (width 0.5) (layer "F.Cu") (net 15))
 (segment (start 104.469138 75.894138) (end 104.45 75.875) (width 0.5) (layer "F.Cu") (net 15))
 (segment (start 105.99 67.685) (end 105.925 67.75) (width 0.3) (layer "F.Cu") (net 15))
 (segment (start 104.469138 95.394959) (end 104.469138 75.894138) (width 0.5) (layer "F.Cu") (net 15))
 (segment (start 104.469138 95.394959) (end 104.469138 97.530862) (width 0.5) (layer "F.Cu") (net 15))
 (segment (start 105.99 55.325) (end 105.99 67.685) (width 0.5) (layer "F.Cu") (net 15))
 (segment (start 105.99 55.325) (end 105.975 55.34) (width 0.3) (layer "F.Cu") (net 15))
 (via (at 105.99 67.685) (size 0.6) (drill 0.3) (layers "F.Cu" "B.Cu") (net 15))
 (via (at 103.375 98.625) (size 0.6) (drill 0.3) (layers "F.Cu" "B.Cu") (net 15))
 (via (at 104.469138 75.894138) (size 0.6) (drill 0.3) (layers "F.Cu" "B.Cu") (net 15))
 (segment (start 104.45 69.225) (end 105.925 67.75) (width 0.5) (layer "B.Cu") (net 15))
 (segment (start 83.005 98.625) (end 79.4 95.02) (width 0.5) (layer "B.Cu") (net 15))
 (segment (start 104.45 75.875) (end 104.45 69.225) (width 0.5) (layer "B.Cu") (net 15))
 (segment (start 103.375 98.625) (end 83.005 98.625) (width 0.5) (layer "B.Cu") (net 15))
 (segment (start 92.425 62.05) (end 87.265108 62.05) (width 0.3) (layer "F.Cu") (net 7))
 (segment (start 82.7 74.225) (end 82.225 74.7) (width 0.3) (layer "F.Cu") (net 7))
 (segment (start 82.7 66.615108) (end 82.7 74.225) (width 0.3) (layer "F.Cu") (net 7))
 (segment (start 87.265108 62.05) (end 82.7 66.615108) (width 0.3) (layer "F.Cu") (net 7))
 (segment (start 82.225 74.7) (end 79.4 74.7) (width 0.3) (layer "F.Cu") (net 7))
 (via (at 92.425 62.05) (size 0.6) (drill 0.3) (layers "F.Cu" "B.Cu") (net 7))
 (segment (start 92.425 62.05) (end 93.275 61.2) (width 0.3) (layer "B.Cu") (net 7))
 (segment (start 93.275 55.555322) (end 93.29 55.555322) (width 0.3) (layer "B.Cu") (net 7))
 (segment (start 93.275 61.2) (end 93.275 55.555322) (width 0.3) (layer "B.Cu") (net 7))
 (segment (start 81.75 69.9) (end 81.75 66.15) (width 0.3) (layer "F.Cu") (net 6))
 (segment (start 81.75 66.15) (end 86.825 61.075) (width 0.3) (layer "F.Cu") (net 6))
 (segment (start 79.49 72.16) (end 81.75 69.9) (width 0.3) (layer "F.Cu") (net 6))
 (segment (start 79.4 72.16) (end 79.49 72.16) (width 0.3) (layer "F.Cu") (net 6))
 (via (at 86.825 61.075) (size 0.6) (drill 0.3) (layers "F.Cu" "B.Cu") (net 6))
 (segment (start 90.75 59.85) (end 90.75 55.325) (width 0.3) (layer "B.Cu") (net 6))
 (segment (start 87 60.9) (end 89.7 60.9) (width 0.3) (layer "B.Cu") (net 6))
 (segment (start 89.7 60.9) (end 90.75 59.85) (width 0.3) (layer "B.Cu") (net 6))
 (segment (start 86.825 61.075) (end 87 60.9) (width 0.3) (layer "B.Cu") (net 6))
 (segment (start 64.7 98.522) (end 63.053 96.875) (width 0.3) (layer "F.Cu") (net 31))
 (segment (start 64.7 102.875) (end 64.7 98.522) (width 0.3) (layer "F.Cu") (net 31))
 (segment (start 61.2 102.875) (end 61.2 98.265) (width 0.3) (layer "F.Cu") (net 33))
 (segment (start 61.2 98.265) (end 59.81 96.875) (width 0.3) (layer "F.Cu") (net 33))
 (segment (start 71.7 102.875) (end 71.7 99.036) (width 0.3) (layer "F.Cu") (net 35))
 (segment (start 71.7 99.036) (end 69.539 96.875) (width 0.3) (layer "F.Cu") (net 35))
 (segment (start 68.2 102.875) (end 68.2 98.779) (width 0.3) (layer "F.Cu") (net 41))
 (segment (start 68.2 98.779) (end 66.296 96.875) (width 0.3) (layer "F.Cu") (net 41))
 (segment (start 65.075 67.775) (end 65.075 83.99) (width 0.3) (layer "F.Cu") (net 32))
 (segment (start 66.26 66.59) (end 65.075 67.775) (width 0.3) (layer "F.Cu") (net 32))
 (segment (start 69.27 66.59) (end 66.26 66.59) (width 0.3) (layer "F.Cu") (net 32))
 (segment (start 65.075 83.99) (end 59.81 89.255) (width 0.3) (layer "F.Cu") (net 32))
 (segment (start 67.445 69.13) (end 65.925 70.65) (width 0.3) (layer "F.Cu") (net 30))
 (segment (start 65.925 70.65) (end 65.925 86.383) (width 0.3) (layer "F.Cu") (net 30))
 (segment (start 65.925 86.383) (end 63.053 89.255) (width 0.3) (layer "F.Cu") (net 30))
 (segment (start 69.27 69.13) (end 67.445 69.13) (width 0.3) (layer "F.Cu") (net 30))
 (segment (start 66.825 72.9) (end 66.825 88.726) (width 0.3) (layer "F.Cu") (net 40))
 (segment (start 66.825 88.726) (end 66.296 89.255) (width 0.3) (layer "F.Cu") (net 40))
 (segment (start 68.055 71.67) (end 66.825 72.9) (width 0.3) (layer "F.Cu") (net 40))
 (segment (start 69.27 71.67) (end 68.055 71.67) (width 0.3) (layer "F.Cu") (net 40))
 (segment (start 67.619 87.335) (end 69.539 89.255) (width 0.3) (layer "F.Cu") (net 34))
 (segment (start 69.27 74.21) (end 67.619 75.861) (width 0.3) (layer "F.Cu") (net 34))
 (segment (start 67.619 75.861) (end 67.619 87.335) (width 0.3) (layer "F.Cu") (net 34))
 (segment (start 72.782 77.832) (end 71.7 76.75) (width 0.3) (layer "F.Cu") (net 38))
 (segment (start 72.782 89.255) (end 72.782 77.832) (width 0.3) (layer "F.Cu") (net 38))
 (segment (start 71.7 76.75) (end 69.27 76.75) (width 0.3) (layer "F.Cu") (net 38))
 (segment (start 70.91 79.29) (end 70.925 79.275) (width 0.3) (layer "F.Cu") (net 36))
 (segment (start 69.27 79.29) (end 70.91 79.29) (width 0.3) (layer "F.Cu") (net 36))
 (via (at 70.925 79.275) (size 0.6) (drill 0.3) (layers "F.Cu" "B.Cu") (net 36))
 (segment (start 70.925 79.275) (end 74.4 79.275) (width 0.3) (layer "B.Cu") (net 36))
 (segment (start 74.4 79.275) (end 75.975 80.85) (width 0.3) (layer "B.Cu") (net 36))
 (segment (start 75.975 88.921387) (end 76.025 88.921387) (width 0.3) (layer "B.Cu") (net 36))
 (segment (start 75.975 80.85) (end 75.975 88.921387) (width 0.3) (layer "B.Cu") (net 36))
 (segment (start 75.2 102.875) (end 75.2 99.293) (width 0.3) (layer "F.Cu") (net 39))
 (segment (start 75.2 99.293) (end 72.782 96.875) (width 0.3) (layer "F.Cu") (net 39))
 (segment (start 78.7 102.875) (end 78.7 99.55) (width 0.3) (layer "F.Cu") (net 37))
 (segment (start 78.7 99.55) (end 76.025 96.875) (width 0.3) (layer "F.Cu") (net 37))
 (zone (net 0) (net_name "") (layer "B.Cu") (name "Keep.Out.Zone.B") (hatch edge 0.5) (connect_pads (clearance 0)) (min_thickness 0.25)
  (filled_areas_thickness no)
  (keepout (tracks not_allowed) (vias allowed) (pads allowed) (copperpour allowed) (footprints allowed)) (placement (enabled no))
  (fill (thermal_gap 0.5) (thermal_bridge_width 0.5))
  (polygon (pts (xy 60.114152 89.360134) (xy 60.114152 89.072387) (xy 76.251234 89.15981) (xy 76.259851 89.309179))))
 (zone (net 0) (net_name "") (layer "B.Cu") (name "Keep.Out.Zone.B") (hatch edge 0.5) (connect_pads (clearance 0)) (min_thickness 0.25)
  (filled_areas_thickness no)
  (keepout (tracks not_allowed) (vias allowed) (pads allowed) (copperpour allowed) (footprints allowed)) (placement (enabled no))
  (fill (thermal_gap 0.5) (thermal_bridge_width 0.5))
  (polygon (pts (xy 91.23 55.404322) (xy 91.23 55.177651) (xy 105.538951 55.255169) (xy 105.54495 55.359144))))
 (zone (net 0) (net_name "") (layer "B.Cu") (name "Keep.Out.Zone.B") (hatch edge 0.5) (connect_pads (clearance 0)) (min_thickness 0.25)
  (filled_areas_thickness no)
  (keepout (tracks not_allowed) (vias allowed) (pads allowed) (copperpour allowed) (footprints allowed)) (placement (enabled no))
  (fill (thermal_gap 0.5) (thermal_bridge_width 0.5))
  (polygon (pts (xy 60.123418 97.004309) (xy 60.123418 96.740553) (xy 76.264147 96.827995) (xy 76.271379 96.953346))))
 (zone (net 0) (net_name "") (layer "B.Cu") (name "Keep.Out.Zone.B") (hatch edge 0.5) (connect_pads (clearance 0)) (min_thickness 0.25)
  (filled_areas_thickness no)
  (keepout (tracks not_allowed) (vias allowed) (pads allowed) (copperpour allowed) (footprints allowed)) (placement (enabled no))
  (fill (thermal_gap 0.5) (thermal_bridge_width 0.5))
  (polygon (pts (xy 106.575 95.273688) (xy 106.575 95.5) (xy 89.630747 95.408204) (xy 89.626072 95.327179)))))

